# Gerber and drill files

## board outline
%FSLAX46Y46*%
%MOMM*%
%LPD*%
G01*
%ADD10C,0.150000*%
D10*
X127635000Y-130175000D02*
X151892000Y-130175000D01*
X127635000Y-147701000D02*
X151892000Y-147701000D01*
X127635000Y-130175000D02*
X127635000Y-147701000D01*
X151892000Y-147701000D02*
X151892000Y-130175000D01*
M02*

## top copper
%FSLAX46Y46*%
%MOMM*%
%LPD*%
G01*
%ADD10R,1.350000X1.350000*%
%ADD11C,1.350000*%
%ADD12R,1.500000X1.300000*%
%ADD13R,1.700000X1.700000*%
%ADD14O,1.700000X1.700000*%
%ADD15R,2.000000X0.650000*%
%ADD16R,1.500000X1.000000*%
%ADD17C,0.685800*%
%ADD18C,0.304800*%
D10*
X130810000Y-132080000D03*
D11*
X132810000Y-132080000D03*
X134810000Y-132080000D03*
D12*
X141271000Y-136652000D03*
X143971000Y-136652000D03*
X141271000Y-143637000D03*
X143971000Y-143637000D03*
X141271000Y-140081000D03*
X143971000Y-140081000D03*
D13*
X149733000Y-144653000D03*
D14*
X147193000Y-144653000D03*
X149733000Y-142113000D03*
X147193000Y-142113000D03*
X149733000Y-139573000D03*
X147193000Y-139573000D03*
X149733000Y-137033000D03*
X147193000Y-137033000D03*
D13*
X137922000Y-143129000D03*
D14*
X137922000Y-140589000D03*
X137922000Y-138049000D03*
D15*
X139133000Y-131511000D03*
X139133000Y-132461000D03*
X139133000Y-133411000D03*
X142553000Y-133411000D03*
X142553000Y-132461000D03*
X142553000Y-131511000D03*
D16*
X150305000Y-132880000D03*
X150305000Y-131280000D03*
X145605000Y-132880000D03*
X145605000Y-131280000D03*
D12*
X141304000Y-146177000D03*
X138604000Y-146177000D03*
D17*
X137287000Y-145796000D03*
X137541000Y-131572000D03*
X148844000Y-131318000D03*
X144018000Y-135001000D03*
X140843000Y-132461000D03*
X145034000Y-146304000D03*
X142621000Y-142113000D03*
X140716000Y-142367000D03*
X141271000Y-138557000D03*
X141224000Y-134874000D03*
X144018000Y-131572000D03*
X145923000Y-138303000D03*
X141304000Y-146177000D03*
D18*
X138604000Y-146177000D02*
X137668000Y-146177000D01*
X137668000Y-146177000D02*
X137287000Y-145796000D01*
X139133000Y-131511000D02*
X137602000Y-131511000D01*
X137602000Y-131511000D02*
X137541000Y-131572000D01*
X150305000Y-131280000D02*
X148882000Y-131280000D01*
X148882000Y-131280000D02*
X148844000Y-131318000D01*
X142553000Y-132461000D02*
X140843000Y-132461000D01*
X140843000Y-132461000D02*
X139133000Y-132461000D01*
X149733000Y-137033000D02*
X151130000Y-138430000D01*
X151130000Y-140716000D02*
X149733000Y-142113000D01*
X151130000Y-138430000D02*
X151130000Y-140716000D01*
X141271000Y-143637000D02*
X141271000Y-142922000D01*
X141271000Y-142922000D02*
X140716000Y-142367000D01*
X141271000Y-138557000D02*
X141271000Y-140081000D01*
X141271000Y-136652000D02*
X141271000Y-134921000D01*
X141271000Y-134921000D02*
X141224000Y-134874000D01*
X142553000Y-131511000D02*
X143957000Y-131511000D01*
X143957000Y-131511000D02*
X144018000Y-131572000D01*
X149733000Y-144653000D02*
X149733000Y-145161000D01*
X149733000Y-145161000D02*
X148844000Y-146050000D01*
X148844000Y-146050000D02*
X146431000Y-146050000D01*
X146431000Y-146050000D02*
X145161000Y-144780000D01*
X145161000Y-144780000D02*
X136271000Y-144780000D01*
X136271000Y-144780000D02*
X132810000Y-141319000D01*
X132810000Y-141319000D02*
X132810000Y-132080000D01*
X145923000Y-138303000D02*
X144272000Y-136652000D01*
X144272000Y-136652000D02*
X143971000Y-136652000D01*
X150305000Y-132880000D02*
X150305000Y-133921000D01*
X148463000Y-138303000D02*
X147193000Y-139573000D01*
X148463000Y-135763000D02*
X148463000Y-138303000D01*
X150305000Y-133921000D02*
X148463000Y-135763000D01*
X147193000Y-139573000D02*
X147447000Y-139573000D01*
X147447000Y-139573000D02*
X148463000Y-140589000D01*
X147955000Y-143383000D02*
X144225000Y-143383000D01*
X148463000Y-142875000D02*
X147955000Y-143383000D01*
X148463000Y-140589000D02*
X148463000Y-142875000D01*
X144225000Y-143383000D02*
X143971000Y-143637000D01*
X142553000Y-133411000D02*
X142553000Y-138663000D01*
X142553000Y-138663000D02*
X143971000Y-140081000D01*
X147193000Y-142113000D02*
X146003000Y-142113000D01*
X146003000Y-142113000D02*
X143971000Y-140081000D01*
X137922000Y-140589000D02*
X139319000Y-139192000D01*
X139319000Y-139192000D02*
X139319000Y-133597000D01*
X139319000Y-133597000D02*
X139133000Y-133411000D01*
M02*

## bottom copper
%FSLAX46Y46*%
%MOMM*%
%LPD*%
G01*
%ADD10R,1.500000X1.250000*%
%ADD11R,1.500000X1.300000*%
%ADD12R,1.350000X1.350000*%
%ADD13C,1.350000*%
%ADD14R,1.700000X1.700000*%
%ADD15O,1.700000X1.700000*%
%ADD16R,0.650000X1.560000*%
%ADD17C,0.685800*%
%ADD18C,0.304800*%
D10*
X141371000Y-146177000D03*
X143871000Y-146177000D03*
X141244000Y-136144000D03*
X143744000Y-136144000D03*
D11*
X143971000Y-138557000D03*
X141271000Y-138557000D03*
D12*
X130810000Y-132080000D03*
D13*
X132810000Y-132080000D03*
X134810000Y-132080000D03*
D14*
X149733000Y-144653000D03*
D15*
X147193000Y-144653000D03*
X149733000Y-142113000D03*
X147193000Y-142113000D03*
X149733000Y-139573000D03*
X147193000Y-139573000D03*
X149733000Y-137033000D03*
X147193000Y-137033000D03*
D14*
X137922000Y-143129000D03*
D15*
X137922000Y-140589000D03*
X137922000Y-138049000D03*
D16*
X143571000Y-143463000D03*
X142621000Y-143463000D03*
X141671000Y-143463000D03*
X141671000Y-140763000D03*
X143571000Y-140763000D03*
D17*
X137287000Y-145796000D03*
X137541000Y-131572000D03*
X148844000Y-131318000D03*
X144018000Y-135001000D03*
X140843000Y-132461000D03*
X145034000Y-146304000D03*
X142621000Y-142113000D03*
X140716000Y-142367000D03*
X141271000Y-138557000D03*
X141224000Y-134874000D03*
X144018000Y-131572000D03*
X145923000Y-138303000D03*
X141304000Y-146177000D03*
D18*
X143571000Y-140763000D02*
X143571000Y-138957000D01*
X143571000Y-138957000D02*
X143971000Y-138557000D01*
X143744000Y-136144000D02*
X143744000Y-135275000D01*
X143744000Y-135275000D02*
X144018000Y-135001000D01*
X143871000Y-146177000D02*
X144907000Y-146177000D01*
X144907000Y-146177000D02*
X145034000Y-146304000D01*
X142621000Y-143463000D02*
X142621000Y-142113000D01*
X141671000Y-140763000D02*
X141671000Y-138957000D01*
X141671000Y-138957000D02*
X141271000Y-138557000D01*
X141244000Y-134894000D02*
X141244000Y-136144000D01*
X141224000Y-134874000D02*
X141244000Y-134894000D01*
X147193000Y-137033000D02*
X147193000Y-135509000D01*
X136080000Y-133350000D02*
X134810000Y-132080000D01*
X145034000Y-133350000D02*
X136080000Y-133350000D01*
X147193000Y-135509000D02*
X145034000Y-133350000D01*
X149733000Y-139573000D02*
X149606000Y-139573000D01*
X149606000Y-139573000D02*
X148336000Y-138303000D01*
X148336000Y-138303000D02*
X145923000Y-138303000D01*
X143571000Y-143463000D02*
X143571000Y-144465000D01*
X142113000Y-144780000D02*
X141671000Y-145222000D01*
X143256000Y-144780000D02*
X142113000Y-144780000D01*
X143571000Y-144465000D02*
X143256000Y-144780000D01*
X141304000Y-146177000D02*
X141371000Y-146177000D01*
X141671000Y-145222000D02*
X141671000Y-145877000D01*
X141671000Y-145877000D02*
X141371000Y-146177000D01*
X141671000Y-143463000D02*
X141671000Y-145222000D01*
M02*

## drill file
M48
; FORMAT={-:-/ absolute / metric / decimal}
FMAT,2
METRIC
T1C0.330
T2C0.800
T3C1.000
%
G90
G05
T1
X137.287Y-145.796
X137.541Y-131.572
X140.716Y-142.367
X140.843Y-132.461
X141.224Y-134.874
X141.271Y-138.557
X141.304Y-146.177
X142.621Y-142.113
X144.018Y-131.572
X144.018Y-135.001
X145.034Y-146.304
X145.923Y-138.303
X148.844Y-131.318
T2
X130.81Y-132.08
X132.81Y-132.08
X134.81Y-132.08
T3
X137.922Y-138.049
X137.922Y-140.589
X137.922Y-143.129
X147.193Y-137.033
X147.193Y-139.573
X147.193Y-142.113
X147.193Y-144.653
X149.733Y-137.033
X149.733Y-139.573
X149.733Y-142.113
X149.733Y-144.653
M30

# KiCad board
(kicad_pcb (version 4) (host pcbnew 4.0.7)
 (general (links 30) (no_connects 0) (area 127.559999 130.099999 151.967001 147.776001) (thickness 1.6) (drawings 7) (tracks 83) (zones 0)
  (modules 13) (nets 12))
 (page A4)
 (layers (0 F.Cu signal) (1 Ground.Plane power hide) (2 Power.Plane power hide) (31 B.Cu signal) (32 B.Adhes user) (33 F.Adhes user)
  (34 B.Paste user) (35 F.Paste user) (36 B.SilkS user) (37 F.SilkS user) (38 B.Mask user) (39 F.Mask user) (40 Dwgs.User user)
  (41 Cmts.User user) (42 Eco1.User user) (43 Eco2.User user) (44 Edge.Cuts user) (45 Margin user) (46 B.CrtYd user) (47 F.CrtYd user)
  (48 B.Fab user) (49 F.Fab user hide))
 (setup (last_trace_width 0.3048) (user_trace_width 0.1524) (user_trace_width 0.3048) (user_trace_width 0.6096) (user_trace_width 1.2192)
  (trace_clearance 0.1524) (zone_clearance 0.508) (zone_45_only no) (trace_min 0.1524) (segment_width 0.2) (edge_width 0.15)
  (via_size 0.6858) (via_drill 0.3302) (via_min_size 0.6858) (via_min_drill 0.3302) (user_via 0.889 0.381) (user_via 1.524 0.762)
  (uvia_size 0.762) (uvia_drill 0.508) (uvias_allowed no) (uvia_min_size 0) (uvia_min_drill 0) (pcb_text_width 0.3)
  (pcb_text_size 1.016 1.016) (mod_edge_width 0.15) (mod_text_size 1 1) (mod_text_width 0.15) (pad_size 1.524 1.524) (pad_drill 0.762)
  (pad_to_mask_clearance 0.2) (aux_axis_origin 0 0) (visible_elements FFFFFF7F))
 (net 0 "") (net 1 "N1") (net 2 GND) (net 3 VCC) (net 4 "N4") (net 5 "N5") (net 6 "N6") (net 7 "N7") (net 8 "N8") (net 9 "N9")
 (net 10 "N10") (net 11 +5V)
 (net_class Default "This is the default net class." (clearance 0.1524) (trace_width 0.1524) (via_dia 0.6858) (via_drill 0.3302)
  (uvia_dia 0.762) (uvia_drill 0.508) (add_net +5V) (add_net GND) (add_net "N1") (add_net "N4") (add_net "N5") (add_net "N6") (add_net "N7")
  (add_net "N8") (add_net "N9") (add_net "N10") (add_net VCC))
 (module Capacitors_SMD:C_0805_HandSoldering (layer B.Cu) (at 142.621 146.177)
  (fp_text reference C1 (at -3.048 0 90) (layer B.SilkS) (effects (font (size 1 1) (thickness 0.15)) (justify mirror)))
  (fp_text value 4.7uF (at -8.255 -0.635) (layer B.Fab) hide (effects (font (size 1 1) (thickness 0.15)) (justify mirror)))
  (pad 1 smd rect (at -1.25 0) (size 1.5 1.25) (layers B.Cu B.Paste B.Mask) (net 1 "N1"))
  (pad 2 smd rect (at 1.25 0) (size 1.5 1.25) (layers B.Cu B.Paste B.Mask) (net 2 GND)))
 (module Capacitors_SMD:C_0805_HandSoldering (layer B.Cu) (at 142.494 136.144)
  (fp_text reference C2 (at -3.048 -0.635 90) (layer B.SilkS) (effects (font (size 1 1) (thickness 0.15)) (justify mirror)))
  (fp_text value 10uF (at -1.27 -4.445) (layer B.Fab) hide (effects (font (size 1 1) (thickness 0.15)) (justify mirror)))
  (pad 1 smd rect (at -1.25 0) (size 1.5 1.25) (layers B.Cu B.Paste B.Mask) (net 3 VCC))
  (pad 2 smd rect (at 1.25 0) (size 1.5 1.25) (layers B.Cu B.Paste B.Mask) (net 2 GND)))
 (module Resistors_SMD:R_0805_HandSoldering (layer B.Cu) (at 142.621 138.557 180)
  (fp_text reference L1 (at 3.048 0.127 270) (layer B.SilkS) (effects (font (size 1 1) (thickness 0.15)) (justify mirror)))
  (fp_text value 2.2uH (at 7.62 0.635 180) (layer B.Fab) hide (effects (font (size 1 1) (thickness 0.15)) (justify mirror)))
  (pad 1 smd rect (at -1.35 0 180) (size 1.5 1.3) (layers B.Cu B.Paste B.Mask) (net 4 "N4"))
  (pad 2 smd rect (at 1.35 0 180) (size 1.5 1.3) (layers B.Cu B.Paste B.Mask) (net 3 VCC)))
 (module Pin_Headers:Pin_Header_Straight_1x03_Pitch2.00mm (layer F.Cu) (at 130.81 132.08 90)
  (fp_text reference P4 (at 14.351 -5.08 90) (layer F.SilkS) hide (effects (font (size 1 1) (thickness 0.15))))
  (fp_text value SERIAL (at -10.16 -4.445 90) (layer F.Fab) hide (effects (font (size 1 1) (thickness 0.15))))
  (pad 1 thru_hole rect (at 0 0 90) (size 1.35 1.35) (drill 0.8) (layers *.Cu *.Mask) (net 2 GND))
  (pad 2 thru_hole circle (at 0 2 90) (size 1.35 1.35) (drill 0.8) (layers *.Cu *.Mask) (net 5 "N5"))
  (pad 3 thru_hole circle (at 0 4 90) (size 1.35 1.35) (drill 0.8) (layers *.Cu *.Mask) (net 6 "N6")))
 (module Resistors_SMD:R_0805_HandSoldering (layer F.Cu) (at 142.621 136.652)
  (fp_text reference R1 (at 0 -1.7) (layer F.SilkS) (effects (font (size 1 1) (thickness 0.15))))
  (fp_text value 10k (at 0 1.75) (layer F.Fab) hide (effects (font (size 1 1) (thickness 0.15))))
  (pad 1 smd rect (at -1.35 0) (size 1.5 1.3) (layers F.Cu F.Paste F.Mask) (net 3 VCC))
  (pad 2 smd rect (at 1.35 0) (size 1.5 1.3) (layers F.Cu F.Paste F.Mask) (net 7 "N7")))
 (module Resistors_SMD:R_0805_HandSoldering (layer F.Cu) (at 142.621 143.637)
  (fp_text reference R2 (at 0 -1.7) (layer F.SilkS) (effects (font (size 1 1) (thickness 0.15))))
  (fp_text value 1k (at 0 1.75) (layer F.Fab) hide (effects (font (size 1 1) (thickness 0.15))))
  (pad 1 smd rect (at -1.35 0) (size 1.5 1.3) (layers F.Cu F.Paste F.Mask) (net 3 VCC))
  (pad 2 smd rect (at 1.35 0) (size 1.5 1.3) (layers F.Cu F.Paste F.Mask) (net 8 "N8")))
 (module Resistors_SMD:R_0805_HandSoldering (layer F.Cu) (at 142.621 140.081)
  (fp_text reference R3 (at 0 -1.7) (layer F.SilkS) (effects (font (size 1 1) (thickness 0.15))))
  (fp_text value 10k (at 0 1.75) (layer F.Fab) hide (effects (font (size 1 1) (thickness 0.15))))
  (pad 1 smd rect (at -1.35 0) (size 1.5 1.3) (layers F.Cu F.Paste F.Mask) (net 3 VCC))
  (pad 2 smd rect (at 1.35 0) (size 1.5 1.3) (layers F.Cu F.Paste F.Mask) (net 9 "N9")))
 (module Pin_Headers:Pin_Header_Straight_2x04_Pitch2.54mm (layer F.Cu) (at 149.733 144.653 180)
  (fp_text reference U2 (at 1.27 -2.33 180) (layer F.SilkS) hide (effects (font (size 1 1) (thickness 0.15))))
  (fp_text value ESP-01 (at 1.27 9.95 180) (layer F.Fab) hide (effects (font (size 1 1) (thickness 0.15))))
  (pad 1 thru_hole rect (at 0 0 180) (size 1.7 1.7) (drill 1) (layers *.Cu *.Mask) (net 5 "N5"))
  (pad 2 thru_hole oval (at 2.54 0 180) (size 1.7 1.7) (drill 1) (layers *.Cu *.Mask) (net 2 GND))
  (pad 3 thru_hole oval (at 0 2.54 180) (size 1.7 1.7) (drill 1) (layers *.Cu *.Mask) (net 3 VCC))
  (pad 4 thru_hole oval (at 2.54 2.54 180) (size 1.7 1.7) (drill 1) (layers *.Cu *.Mask) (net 9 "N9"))
  (pad 5 thru_hole oval (at 0 5.08 180) (size 1.7 1.7) (drill 1) (layers *.Cu *.Mask) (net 7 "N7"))
  (pad 6 thru_hole oval (at 2.54 5.08 180) (size 1.7 1.7) (drill 1) (layers *.Cu *.Mask) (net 8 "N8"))
  (pad 7 thru_hole oval (at 0 7.62 180) (size 1.7 1.7) (drill 1) (layers *.Cu *.Mask) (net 3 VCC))
  (pad 8 thru_hole oval (at 2.54 7.62 180) (size 1.7 1.7) (drill 1) (layers *.Cu *.Mask) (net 6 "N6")))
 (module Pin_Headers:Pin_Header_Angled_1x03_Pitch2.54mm (layer F.Cu) (at 137.922 143.129 180)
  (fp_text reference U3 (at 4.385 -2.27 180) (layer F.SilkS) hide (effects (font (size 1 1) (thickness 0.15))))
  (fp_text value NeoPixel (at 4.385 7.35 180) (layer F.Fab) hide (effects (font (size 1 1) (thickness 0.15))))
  (pad 1 thru_hole rect (at 0 0 180) (size 1.7 1.7) (drill 1) (layers *.Cu *.Mask) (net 2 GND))
  (pad 2 thru_hole oval (at 0 2.54 180) (size 1.7 1.7) (drill 1) (layers *.Cu *.Mask) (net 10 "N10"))
  (pad 3 thru_hole oval (at 0 5.08 180) (size 1.7 1.7) (drill 1) (layers *.Cu *.Mask) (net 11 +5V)))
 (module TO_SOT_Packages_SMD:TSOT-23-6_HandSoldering (layer F.Cu) (at 140.843 132.461)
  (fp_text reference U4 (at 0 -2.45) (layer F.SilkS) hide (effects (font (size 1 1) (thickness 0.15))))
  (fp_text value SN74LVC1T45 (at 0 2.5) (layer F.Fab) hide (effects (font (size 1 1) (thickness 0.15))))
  (pad 1 smd rect (at -1.71 -0.95) (size 2 0.65) (layers F.Cu F.Paste F.Mask) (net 11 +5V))
  (pad 2 smd rect (at -1.71 0) (size 2 0.65) (layers F.Cu F.Paste F.Mask) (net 2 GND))
  (pad 3 smd rect (at -1.71 0.95) (size 2 0.65) (layers F.Cu F.Paste F.Mask) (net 10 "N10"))
  (pad 4 smd rect (at 1.71 0.95) (size 2 0.65) (layers F.Cu F.Paste F.Mask) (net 9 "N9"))
  (pad 5 smd rect (at 1.71 0) (size 2 0.65) (layers F.Cu F.Paste F.Mask) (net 2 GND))
  (pad 6 smd rect (at 1.71 -0.95) (size 2 0.65) (layers F.Cu F.Paste F.Mask) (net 3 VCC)))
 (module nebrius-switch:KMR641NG (layer F.Cu) (at 147.955 132.08 180)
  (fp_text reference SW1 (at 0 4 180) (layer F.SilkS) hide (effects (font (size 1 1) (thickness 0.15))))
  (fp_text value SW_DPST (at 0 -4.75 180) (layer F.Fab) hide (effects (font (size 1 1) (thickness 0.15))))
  (pad 1 smd rect (at -2.35 -0.8 180) (size 1.5 1) (layers F.Cu F.Paste F.Mask) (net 8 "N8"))
  (pad 2 smd rect (at -2.35 0.8 180) (size 1.5 1) (layers F.Cu F.Paste F.Mask) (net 2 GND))
  (pad 3 smd rect (at 2.35 -0.8 180) (size 1.5 1) (layers F.Cu F.Paste F.Mask))
  (pad 4 smd rect (at 2.35 0.8 180) (size 1.5 1) (layers F.Cu F.Paste F.Mask)))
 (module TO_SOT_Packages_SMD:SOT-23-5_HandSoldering (layer B.Cu) (at 142.621 142.113 90)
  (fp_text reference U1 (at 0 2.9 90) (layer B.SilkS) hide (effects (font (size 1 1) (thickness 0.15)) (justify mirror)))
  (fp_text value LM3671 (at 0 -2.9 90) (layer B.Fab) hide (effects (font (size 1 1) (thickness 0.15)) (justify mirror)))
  (pad 1 smd rect (at -1.35 0.95 90) (size 1.56 0.65) (layers B.Cu B.Paste B.Mask) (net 1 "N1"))
  (pad 2 smd rect (at -1.35 0 90) (size 1.56 0.65) (layers B.Cu B.Paste B.Mask) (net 2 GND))
  (pad 3 smd rect (at -1.35 -0.95 90) (size 1.56 0.65) (layers B.Cu B.Paste B.Mask) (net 1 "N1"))
  (pad 4 smd rect (at 1.35 -0.95 90) (size 1.56 0.65) (layers B.Cu B.Paste B.Mask) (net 3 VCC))
  (pad 5 smd rect (at 1.35 0.95 90) (size 1.56 0.65) (layers B.Cu B.Paste B.Mask) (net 4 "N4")))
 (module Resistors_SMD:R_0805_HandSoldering (layer F.Cu) (at 139.954 146.177 180)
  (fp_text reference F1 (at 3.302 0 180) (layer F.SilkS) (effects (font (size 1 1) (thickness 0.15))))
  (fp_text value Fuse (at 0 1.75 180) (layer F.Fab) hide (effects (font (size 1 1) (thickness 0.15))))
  (pad 1 smd rect (at -1.35 0 180) (size 1.5 1.3) (layers F.Cu F.Paste F.Mask) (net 1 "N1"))
  (pad 2 smd rect (at 1.35 0 180) (size 1.5 1.3) (layers F.Cu F.Paste F.Mask) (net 11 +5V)))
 (gr_line (start 127.635 130.175) (end 151.892 130.175) (angle 90) (layer Edge.Cuts) (width 0.15))
 (gr_line (start 127.635 147.701) (end 151.892 147.701) (angle 90) (layer Edge.Cuts) (width 0.15))
 (gr_line (start 127.635 130.175) (end 127.635 147.701) (angle 90) (layer Edge.Cuts) (width 0.15))
 (gr_line (start 151.892 147.701) (end 151.892 130.175) (angle 90) (layer Edge.Cuts) (width 0.15))
 (segment (start 143.571 140.763) (end 143.571 138.957) (width 0.3048) (layer B.Cu) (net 4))
 (segment (start 143.571 138.957) (end 143.971 138.557) (width 0.3048) (layer B.Cu) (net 4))
 (segment (start 138.604 146.177) (end 137.668 146.177) (width 0.3048) (layer F.Cu) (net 11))
 (via (at 137.287 145.796) (size 0.6858) (drill 0.3302) (layers F.Cu B.Cu) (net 11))
 (segment (start 137.668 146.177) (end 137.287 145.796) (width 0.3048) (layer F.Cu) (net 11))
 (segment (start 139.133 131.511) (end 137.602 131.511) (width 0.3048) (layer F.Cu) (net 11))
 (via (at 137.541 131.572) (size 0.6858) (drill 0.3302) (layers F.Cu B.Cu) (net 11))
 (segment (start 137.602 131.511) (end 137.541 131.572) (width 0.3048) (layer F.Cu) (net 11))
 (segment (start 150.305 131.28) (end 148.882 131.28) (width 0.3048) (layer F.Cu) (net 2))
 (via (at 148.844 131.318) (size 0.6858) (drill 0.3302) (layers F.Cu B.Cu) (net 2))
 (segment (start 148.882 131.28) (end 148.844 131.318) (width 0.3048) (layer F.Cu) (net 2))
 (segment (start 143.744 136.144) (end 143.744 135.275) (width 0.3048) (layer B.Cu) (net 2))
 (via (at 144.018 135.001) (size 0.6858) (drill 0.3302) (layers F.Cu B.Cu) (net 2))
 (segment (start 143.744 135.275) (end 144.018 135.001) (width 0.3048) (layer B.Cu) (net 2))
 (segment (start 142.553 132.461) (end 140.843 132.461) (width 0.3048) (layer F.Cu) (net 2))
 (via (at 140.843 132.461) (size 0.6858) (drill 0.3302) (layers F.Cu B.Cu) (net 2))
 (segment (start 140.843 132.461) (end 139.133 132.461) (width 0.3048) (layer F.Cu) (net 2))
 (segment (start 143.871 146.177) (end 144.907 146.177) (width 0.3048) (layer B.Cu) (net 2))
 (via (at 145.034 146.304) (size 0.6858) (drill 0.3302) (layers F.Cu B.Cu) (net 2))
 (segment (start 144.907 146.177) (end 145.034 146.304) (width 0.3048) (layer B.Cu) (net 2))
 (segment (start 142.621 143.463) (end 142.621 142.113) (width 0.3048) (layer B.Cu) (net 2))
 (via (at 142.621 142.113) (size 0.6858) (drill 0.3302) (layers F.Cu B.Cu) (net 2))
 (segment (start 149.733 137.033) (end 151.13 138.43) (width 0.3048) (layer F.Cu) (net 3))
 (segment (start 151.13 140.716) (end 149.733 142.113) (width 0.3048) (layer F.Cu) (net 3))
 (segment (start 151.13 138.43) (end 151.13 140.716) (width 0.3048) (layer F.Cu) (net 3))
 (segment (start 141.271 143.637) (end 141.271 142.922) (width 0.3048) (layer F.Cu) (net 3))
 (via (at 140.716 142.367) (size 0.6858) (drill 0.3302) (layers F.Cu B.Cu) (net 3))
 (segment (start 141.271 142.922) (end 140.716 142.367) (width 0.3048) (layer F.Cu) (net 3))
 (segment (start 141.671 140.763) (end 141.671 138.957) (width 0.3048) (layer B.Cu) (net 3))
 (segment (start 141.671 138.957) (end 141.271 138.557) (width 0.3048) (layer B.Cu) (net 3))
 (via (at 141.271 138.557) (size 0.6858) (drill 0.3302) (layers F.Cu B.Cu) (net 3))
 (segment (start 141.271 138.557) (end 141.271 140.081) (width 0.3048) (layer F.Cu) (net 3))
 (segment (start 141.271 136.652) (end 141.271 134.921) (width 0.3048) (layer F.Cu) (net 3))
 (segment (start 141.244 134.894) (end 141.244 136.144) (width 0.3048) (layer B.Cu) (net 3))
 (segment (start 141.224 134.874) (end 141.244 134.894) (width 0.3048) (layer B.Cu) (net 3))
 (via (at 141.224 134.874) (size 0.6858) (drill 0.3302) (layers F.Cu B.Cu) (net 3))
 (segment (start 141.271 134.921) (end 141.224 134.874) (width 0.3048) (layer F.Cu) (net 3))
 (segment (start 142.553 131.511) (end 143.957 131.511) (width 0.3048) (layer F.Cu) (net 3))
 (via (at 144.018 131.572) (size 0.6858) (drill 0.3302) (layers F.Cu B.Cu) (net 3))
 (segment (start 143.957 131.511) (end 144.018 131.572) (width 0.3048) (layer F.Cu) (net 3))
 (segment (start 149.733 144.653) (end 149.733 145.161) (width 0.3048) (layer F.Cu) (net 5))
 (segment (start 149.733 145.161) (end 148.844 146.05) (width 0.3048) (layer F.Cu) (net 5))
 (segment (start 148.844 146.05) (end 146.431 146.05) (width 0.3048) (layer F.Cu) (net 5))
 (segment (start 146.431 146.05) (end 145.161 144.78) (width 0.3048) (layer F.Cu) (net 5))
 (segment (start 145.161 144.78) (end 136.271 144.78) (width 0.3048) (layer F.Cu) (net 5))
 (segment (start 136.271 144.78) (end 132.81 141.319) (width 0.3048) (layer F.Cu) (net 5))
 (segment (start 132.81 141.319) (end 132.81 132.08) (width 0.3048) (layer F.Cu) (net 5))
 (segment (start 147.193 137.033) (end 147.193 135.509) (width 0.3048) (layer B.Cu) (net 6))
 (segment (start 136.08 133.35) (end 134.81 132.08) (width 0.3048) (layer B.Cu) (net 6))
 (segment (start 145.034 133.35) (end 136.08 133.35) (width 0.3048) (layer B.Cu) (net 6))
 (segment (start 147.193 135.509) (end 145.034 133.35) (width 0.3048) (layer B.Cu) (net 6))
 (segment (start 149.733 139.573) (end 149.606 139.573) (width 0.3048) (layer B.Cu) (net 7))
 (segment (start 149.606 139.573) (end 148.336 138.303) (width 0.3048) (layer B.Cu) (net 7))
 (segment (start 148.336 138.303) (end 145.923 138.303) (width 0.3048) (layer B.Cu) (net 7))
 (via (at 145.923 138.303) (size 0.6858) (drill 0.3302) (layers F.Cu B.Cu) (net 7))
 (segment (start 145.923 138.303) (end 144.272 136.652) (width 0.3048) (layer F.Cu) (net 7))
 (segment (start 144.272 136.652) (end 143.971 136.652) (width 0.3048) (layer F.Cu) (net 7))
 (segment (start 150.305 132.88) (end 150.305 133.921) (width 0.3048) (layer F.Cu) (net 8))
 (segment (start 148.463 138.303) (end 147.193 139.573) (width 0.3048) (layer F.Cu) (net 8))
 (segment (start 148.463 135.763) (end 148.463 138.303) (width 0.3048) (layer F.Cu) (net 8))
 (segment (start 150.305 133.921) (end 148.463 135.763) (width 0.3048) (layer F.Cu) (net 8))
 (segment (start 147.193 139.573) (end 147.447 139.573) (width 0.3048) (layer F.Cu) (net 8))
 (segment (start 147.447 139.573) (end 148.463 140.589) (width 0.3048) (layer F.Cu) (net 8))
 (segment (start 147.955 143.383) (end 144.225 143.383) (width 0.3048) (layer F.Cu) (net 8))
 (segment (start 148.463 142.875) (end 147.955 143.383) (width 0.3048) (layer F.Cu) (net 8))
 (segment (start 148.463 140.589) (end 148.463 142.875) (width 0.3048) (layer F.Cu) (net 8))
 (segment (start 144.225 143.383) (end 143.971 143.637) (width 0.3048) (layer F.Cu) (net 8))
 (segment (start 142.553 133.411) (end 142.553 138.663) (width 0.3048) (layer F.Cu) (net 9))
 (segment (start 142.553 138.663) (end 143.971 140.081) (width 0.3048) (layer F.Cu) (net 9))
 (segment (start 147.193 142.113) (end 146.003 142.113) (width 0.3048) (layer F.Cu) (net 9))
 (segment (start 146.003 142.113) (end 143.971 140.081) (width 0.3048) (layer F.Cu) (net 9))
 (segment (start 137.922 140.589) (end 139.319 139.192) (width 0.3048) (layer F.Cu) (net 10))
 (segment (start 139.319 139.192) (end 139.319 133.597) (width 0.3048) (layer F.Cu) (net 10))
 (segment (start 139.319 133.597) (end 139.133 133.411) (width 0.3048) (layer F.Cu) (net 10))
 (segment (start 143.571 143.463) (end 143.571 144.465) (width 0.3048) (layer B.Cu) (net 1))
 (segment (start 142.113 144.78) (end 141.671 145.222) (width 0.3048) (layer B.Cu) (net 1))
 (segment (start 143.256 144.78) (end 142.113 144.78) (width 0.3048) (layer B.Cu) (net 1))
 (segment (start 143.571 144.465) (end 143.256 144.78) (width 0.3048) (layer B.Cu) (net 1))
 (via (at 141.304 146.177) (size 0.6858) (drill 0.3302) (layers F.Cu B.Cu) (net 1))
 (segment (start 141.304 146.177) (end 141.371 146.177) (width 0.3048) (layer B.Cu) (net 1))
 (segment (start 141.671 145.222) (end 141.671 145.877) (width 0.3048) (layer B.Cu) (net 1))
 (segment (start 141.671 145.877) (end 141.371 146.177) (width 0.3048) (layer B.Cu) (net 1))
 (segment (start 141.671 143.463) (end 141.671 145.222) (width 0.3048) (layer B.Cu) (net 1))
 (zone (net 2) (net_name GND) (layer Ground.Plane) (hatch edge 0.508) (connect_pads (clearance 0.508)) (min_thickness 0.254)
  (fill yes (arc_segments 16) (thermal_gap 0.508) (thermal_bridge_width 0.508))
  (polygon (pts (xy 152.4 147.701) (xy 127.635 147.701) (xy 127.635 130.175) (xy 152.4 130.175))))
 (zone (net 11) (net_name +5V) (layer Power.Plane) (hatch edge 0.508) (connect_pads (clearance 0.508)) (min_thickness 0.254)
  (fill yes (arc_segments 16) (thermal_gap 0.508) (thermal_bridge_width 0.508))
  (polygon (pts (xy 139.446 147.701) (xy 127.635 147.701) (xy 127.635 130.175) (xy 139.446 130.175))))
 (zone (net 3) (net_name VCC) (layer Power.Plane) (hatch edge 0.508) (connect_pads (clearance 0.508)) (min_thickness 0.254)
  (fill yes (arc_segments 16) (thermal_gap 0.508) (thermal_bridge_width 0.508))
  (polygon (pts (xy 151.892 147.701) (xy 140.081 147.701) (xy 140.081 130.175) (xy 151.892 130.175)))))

